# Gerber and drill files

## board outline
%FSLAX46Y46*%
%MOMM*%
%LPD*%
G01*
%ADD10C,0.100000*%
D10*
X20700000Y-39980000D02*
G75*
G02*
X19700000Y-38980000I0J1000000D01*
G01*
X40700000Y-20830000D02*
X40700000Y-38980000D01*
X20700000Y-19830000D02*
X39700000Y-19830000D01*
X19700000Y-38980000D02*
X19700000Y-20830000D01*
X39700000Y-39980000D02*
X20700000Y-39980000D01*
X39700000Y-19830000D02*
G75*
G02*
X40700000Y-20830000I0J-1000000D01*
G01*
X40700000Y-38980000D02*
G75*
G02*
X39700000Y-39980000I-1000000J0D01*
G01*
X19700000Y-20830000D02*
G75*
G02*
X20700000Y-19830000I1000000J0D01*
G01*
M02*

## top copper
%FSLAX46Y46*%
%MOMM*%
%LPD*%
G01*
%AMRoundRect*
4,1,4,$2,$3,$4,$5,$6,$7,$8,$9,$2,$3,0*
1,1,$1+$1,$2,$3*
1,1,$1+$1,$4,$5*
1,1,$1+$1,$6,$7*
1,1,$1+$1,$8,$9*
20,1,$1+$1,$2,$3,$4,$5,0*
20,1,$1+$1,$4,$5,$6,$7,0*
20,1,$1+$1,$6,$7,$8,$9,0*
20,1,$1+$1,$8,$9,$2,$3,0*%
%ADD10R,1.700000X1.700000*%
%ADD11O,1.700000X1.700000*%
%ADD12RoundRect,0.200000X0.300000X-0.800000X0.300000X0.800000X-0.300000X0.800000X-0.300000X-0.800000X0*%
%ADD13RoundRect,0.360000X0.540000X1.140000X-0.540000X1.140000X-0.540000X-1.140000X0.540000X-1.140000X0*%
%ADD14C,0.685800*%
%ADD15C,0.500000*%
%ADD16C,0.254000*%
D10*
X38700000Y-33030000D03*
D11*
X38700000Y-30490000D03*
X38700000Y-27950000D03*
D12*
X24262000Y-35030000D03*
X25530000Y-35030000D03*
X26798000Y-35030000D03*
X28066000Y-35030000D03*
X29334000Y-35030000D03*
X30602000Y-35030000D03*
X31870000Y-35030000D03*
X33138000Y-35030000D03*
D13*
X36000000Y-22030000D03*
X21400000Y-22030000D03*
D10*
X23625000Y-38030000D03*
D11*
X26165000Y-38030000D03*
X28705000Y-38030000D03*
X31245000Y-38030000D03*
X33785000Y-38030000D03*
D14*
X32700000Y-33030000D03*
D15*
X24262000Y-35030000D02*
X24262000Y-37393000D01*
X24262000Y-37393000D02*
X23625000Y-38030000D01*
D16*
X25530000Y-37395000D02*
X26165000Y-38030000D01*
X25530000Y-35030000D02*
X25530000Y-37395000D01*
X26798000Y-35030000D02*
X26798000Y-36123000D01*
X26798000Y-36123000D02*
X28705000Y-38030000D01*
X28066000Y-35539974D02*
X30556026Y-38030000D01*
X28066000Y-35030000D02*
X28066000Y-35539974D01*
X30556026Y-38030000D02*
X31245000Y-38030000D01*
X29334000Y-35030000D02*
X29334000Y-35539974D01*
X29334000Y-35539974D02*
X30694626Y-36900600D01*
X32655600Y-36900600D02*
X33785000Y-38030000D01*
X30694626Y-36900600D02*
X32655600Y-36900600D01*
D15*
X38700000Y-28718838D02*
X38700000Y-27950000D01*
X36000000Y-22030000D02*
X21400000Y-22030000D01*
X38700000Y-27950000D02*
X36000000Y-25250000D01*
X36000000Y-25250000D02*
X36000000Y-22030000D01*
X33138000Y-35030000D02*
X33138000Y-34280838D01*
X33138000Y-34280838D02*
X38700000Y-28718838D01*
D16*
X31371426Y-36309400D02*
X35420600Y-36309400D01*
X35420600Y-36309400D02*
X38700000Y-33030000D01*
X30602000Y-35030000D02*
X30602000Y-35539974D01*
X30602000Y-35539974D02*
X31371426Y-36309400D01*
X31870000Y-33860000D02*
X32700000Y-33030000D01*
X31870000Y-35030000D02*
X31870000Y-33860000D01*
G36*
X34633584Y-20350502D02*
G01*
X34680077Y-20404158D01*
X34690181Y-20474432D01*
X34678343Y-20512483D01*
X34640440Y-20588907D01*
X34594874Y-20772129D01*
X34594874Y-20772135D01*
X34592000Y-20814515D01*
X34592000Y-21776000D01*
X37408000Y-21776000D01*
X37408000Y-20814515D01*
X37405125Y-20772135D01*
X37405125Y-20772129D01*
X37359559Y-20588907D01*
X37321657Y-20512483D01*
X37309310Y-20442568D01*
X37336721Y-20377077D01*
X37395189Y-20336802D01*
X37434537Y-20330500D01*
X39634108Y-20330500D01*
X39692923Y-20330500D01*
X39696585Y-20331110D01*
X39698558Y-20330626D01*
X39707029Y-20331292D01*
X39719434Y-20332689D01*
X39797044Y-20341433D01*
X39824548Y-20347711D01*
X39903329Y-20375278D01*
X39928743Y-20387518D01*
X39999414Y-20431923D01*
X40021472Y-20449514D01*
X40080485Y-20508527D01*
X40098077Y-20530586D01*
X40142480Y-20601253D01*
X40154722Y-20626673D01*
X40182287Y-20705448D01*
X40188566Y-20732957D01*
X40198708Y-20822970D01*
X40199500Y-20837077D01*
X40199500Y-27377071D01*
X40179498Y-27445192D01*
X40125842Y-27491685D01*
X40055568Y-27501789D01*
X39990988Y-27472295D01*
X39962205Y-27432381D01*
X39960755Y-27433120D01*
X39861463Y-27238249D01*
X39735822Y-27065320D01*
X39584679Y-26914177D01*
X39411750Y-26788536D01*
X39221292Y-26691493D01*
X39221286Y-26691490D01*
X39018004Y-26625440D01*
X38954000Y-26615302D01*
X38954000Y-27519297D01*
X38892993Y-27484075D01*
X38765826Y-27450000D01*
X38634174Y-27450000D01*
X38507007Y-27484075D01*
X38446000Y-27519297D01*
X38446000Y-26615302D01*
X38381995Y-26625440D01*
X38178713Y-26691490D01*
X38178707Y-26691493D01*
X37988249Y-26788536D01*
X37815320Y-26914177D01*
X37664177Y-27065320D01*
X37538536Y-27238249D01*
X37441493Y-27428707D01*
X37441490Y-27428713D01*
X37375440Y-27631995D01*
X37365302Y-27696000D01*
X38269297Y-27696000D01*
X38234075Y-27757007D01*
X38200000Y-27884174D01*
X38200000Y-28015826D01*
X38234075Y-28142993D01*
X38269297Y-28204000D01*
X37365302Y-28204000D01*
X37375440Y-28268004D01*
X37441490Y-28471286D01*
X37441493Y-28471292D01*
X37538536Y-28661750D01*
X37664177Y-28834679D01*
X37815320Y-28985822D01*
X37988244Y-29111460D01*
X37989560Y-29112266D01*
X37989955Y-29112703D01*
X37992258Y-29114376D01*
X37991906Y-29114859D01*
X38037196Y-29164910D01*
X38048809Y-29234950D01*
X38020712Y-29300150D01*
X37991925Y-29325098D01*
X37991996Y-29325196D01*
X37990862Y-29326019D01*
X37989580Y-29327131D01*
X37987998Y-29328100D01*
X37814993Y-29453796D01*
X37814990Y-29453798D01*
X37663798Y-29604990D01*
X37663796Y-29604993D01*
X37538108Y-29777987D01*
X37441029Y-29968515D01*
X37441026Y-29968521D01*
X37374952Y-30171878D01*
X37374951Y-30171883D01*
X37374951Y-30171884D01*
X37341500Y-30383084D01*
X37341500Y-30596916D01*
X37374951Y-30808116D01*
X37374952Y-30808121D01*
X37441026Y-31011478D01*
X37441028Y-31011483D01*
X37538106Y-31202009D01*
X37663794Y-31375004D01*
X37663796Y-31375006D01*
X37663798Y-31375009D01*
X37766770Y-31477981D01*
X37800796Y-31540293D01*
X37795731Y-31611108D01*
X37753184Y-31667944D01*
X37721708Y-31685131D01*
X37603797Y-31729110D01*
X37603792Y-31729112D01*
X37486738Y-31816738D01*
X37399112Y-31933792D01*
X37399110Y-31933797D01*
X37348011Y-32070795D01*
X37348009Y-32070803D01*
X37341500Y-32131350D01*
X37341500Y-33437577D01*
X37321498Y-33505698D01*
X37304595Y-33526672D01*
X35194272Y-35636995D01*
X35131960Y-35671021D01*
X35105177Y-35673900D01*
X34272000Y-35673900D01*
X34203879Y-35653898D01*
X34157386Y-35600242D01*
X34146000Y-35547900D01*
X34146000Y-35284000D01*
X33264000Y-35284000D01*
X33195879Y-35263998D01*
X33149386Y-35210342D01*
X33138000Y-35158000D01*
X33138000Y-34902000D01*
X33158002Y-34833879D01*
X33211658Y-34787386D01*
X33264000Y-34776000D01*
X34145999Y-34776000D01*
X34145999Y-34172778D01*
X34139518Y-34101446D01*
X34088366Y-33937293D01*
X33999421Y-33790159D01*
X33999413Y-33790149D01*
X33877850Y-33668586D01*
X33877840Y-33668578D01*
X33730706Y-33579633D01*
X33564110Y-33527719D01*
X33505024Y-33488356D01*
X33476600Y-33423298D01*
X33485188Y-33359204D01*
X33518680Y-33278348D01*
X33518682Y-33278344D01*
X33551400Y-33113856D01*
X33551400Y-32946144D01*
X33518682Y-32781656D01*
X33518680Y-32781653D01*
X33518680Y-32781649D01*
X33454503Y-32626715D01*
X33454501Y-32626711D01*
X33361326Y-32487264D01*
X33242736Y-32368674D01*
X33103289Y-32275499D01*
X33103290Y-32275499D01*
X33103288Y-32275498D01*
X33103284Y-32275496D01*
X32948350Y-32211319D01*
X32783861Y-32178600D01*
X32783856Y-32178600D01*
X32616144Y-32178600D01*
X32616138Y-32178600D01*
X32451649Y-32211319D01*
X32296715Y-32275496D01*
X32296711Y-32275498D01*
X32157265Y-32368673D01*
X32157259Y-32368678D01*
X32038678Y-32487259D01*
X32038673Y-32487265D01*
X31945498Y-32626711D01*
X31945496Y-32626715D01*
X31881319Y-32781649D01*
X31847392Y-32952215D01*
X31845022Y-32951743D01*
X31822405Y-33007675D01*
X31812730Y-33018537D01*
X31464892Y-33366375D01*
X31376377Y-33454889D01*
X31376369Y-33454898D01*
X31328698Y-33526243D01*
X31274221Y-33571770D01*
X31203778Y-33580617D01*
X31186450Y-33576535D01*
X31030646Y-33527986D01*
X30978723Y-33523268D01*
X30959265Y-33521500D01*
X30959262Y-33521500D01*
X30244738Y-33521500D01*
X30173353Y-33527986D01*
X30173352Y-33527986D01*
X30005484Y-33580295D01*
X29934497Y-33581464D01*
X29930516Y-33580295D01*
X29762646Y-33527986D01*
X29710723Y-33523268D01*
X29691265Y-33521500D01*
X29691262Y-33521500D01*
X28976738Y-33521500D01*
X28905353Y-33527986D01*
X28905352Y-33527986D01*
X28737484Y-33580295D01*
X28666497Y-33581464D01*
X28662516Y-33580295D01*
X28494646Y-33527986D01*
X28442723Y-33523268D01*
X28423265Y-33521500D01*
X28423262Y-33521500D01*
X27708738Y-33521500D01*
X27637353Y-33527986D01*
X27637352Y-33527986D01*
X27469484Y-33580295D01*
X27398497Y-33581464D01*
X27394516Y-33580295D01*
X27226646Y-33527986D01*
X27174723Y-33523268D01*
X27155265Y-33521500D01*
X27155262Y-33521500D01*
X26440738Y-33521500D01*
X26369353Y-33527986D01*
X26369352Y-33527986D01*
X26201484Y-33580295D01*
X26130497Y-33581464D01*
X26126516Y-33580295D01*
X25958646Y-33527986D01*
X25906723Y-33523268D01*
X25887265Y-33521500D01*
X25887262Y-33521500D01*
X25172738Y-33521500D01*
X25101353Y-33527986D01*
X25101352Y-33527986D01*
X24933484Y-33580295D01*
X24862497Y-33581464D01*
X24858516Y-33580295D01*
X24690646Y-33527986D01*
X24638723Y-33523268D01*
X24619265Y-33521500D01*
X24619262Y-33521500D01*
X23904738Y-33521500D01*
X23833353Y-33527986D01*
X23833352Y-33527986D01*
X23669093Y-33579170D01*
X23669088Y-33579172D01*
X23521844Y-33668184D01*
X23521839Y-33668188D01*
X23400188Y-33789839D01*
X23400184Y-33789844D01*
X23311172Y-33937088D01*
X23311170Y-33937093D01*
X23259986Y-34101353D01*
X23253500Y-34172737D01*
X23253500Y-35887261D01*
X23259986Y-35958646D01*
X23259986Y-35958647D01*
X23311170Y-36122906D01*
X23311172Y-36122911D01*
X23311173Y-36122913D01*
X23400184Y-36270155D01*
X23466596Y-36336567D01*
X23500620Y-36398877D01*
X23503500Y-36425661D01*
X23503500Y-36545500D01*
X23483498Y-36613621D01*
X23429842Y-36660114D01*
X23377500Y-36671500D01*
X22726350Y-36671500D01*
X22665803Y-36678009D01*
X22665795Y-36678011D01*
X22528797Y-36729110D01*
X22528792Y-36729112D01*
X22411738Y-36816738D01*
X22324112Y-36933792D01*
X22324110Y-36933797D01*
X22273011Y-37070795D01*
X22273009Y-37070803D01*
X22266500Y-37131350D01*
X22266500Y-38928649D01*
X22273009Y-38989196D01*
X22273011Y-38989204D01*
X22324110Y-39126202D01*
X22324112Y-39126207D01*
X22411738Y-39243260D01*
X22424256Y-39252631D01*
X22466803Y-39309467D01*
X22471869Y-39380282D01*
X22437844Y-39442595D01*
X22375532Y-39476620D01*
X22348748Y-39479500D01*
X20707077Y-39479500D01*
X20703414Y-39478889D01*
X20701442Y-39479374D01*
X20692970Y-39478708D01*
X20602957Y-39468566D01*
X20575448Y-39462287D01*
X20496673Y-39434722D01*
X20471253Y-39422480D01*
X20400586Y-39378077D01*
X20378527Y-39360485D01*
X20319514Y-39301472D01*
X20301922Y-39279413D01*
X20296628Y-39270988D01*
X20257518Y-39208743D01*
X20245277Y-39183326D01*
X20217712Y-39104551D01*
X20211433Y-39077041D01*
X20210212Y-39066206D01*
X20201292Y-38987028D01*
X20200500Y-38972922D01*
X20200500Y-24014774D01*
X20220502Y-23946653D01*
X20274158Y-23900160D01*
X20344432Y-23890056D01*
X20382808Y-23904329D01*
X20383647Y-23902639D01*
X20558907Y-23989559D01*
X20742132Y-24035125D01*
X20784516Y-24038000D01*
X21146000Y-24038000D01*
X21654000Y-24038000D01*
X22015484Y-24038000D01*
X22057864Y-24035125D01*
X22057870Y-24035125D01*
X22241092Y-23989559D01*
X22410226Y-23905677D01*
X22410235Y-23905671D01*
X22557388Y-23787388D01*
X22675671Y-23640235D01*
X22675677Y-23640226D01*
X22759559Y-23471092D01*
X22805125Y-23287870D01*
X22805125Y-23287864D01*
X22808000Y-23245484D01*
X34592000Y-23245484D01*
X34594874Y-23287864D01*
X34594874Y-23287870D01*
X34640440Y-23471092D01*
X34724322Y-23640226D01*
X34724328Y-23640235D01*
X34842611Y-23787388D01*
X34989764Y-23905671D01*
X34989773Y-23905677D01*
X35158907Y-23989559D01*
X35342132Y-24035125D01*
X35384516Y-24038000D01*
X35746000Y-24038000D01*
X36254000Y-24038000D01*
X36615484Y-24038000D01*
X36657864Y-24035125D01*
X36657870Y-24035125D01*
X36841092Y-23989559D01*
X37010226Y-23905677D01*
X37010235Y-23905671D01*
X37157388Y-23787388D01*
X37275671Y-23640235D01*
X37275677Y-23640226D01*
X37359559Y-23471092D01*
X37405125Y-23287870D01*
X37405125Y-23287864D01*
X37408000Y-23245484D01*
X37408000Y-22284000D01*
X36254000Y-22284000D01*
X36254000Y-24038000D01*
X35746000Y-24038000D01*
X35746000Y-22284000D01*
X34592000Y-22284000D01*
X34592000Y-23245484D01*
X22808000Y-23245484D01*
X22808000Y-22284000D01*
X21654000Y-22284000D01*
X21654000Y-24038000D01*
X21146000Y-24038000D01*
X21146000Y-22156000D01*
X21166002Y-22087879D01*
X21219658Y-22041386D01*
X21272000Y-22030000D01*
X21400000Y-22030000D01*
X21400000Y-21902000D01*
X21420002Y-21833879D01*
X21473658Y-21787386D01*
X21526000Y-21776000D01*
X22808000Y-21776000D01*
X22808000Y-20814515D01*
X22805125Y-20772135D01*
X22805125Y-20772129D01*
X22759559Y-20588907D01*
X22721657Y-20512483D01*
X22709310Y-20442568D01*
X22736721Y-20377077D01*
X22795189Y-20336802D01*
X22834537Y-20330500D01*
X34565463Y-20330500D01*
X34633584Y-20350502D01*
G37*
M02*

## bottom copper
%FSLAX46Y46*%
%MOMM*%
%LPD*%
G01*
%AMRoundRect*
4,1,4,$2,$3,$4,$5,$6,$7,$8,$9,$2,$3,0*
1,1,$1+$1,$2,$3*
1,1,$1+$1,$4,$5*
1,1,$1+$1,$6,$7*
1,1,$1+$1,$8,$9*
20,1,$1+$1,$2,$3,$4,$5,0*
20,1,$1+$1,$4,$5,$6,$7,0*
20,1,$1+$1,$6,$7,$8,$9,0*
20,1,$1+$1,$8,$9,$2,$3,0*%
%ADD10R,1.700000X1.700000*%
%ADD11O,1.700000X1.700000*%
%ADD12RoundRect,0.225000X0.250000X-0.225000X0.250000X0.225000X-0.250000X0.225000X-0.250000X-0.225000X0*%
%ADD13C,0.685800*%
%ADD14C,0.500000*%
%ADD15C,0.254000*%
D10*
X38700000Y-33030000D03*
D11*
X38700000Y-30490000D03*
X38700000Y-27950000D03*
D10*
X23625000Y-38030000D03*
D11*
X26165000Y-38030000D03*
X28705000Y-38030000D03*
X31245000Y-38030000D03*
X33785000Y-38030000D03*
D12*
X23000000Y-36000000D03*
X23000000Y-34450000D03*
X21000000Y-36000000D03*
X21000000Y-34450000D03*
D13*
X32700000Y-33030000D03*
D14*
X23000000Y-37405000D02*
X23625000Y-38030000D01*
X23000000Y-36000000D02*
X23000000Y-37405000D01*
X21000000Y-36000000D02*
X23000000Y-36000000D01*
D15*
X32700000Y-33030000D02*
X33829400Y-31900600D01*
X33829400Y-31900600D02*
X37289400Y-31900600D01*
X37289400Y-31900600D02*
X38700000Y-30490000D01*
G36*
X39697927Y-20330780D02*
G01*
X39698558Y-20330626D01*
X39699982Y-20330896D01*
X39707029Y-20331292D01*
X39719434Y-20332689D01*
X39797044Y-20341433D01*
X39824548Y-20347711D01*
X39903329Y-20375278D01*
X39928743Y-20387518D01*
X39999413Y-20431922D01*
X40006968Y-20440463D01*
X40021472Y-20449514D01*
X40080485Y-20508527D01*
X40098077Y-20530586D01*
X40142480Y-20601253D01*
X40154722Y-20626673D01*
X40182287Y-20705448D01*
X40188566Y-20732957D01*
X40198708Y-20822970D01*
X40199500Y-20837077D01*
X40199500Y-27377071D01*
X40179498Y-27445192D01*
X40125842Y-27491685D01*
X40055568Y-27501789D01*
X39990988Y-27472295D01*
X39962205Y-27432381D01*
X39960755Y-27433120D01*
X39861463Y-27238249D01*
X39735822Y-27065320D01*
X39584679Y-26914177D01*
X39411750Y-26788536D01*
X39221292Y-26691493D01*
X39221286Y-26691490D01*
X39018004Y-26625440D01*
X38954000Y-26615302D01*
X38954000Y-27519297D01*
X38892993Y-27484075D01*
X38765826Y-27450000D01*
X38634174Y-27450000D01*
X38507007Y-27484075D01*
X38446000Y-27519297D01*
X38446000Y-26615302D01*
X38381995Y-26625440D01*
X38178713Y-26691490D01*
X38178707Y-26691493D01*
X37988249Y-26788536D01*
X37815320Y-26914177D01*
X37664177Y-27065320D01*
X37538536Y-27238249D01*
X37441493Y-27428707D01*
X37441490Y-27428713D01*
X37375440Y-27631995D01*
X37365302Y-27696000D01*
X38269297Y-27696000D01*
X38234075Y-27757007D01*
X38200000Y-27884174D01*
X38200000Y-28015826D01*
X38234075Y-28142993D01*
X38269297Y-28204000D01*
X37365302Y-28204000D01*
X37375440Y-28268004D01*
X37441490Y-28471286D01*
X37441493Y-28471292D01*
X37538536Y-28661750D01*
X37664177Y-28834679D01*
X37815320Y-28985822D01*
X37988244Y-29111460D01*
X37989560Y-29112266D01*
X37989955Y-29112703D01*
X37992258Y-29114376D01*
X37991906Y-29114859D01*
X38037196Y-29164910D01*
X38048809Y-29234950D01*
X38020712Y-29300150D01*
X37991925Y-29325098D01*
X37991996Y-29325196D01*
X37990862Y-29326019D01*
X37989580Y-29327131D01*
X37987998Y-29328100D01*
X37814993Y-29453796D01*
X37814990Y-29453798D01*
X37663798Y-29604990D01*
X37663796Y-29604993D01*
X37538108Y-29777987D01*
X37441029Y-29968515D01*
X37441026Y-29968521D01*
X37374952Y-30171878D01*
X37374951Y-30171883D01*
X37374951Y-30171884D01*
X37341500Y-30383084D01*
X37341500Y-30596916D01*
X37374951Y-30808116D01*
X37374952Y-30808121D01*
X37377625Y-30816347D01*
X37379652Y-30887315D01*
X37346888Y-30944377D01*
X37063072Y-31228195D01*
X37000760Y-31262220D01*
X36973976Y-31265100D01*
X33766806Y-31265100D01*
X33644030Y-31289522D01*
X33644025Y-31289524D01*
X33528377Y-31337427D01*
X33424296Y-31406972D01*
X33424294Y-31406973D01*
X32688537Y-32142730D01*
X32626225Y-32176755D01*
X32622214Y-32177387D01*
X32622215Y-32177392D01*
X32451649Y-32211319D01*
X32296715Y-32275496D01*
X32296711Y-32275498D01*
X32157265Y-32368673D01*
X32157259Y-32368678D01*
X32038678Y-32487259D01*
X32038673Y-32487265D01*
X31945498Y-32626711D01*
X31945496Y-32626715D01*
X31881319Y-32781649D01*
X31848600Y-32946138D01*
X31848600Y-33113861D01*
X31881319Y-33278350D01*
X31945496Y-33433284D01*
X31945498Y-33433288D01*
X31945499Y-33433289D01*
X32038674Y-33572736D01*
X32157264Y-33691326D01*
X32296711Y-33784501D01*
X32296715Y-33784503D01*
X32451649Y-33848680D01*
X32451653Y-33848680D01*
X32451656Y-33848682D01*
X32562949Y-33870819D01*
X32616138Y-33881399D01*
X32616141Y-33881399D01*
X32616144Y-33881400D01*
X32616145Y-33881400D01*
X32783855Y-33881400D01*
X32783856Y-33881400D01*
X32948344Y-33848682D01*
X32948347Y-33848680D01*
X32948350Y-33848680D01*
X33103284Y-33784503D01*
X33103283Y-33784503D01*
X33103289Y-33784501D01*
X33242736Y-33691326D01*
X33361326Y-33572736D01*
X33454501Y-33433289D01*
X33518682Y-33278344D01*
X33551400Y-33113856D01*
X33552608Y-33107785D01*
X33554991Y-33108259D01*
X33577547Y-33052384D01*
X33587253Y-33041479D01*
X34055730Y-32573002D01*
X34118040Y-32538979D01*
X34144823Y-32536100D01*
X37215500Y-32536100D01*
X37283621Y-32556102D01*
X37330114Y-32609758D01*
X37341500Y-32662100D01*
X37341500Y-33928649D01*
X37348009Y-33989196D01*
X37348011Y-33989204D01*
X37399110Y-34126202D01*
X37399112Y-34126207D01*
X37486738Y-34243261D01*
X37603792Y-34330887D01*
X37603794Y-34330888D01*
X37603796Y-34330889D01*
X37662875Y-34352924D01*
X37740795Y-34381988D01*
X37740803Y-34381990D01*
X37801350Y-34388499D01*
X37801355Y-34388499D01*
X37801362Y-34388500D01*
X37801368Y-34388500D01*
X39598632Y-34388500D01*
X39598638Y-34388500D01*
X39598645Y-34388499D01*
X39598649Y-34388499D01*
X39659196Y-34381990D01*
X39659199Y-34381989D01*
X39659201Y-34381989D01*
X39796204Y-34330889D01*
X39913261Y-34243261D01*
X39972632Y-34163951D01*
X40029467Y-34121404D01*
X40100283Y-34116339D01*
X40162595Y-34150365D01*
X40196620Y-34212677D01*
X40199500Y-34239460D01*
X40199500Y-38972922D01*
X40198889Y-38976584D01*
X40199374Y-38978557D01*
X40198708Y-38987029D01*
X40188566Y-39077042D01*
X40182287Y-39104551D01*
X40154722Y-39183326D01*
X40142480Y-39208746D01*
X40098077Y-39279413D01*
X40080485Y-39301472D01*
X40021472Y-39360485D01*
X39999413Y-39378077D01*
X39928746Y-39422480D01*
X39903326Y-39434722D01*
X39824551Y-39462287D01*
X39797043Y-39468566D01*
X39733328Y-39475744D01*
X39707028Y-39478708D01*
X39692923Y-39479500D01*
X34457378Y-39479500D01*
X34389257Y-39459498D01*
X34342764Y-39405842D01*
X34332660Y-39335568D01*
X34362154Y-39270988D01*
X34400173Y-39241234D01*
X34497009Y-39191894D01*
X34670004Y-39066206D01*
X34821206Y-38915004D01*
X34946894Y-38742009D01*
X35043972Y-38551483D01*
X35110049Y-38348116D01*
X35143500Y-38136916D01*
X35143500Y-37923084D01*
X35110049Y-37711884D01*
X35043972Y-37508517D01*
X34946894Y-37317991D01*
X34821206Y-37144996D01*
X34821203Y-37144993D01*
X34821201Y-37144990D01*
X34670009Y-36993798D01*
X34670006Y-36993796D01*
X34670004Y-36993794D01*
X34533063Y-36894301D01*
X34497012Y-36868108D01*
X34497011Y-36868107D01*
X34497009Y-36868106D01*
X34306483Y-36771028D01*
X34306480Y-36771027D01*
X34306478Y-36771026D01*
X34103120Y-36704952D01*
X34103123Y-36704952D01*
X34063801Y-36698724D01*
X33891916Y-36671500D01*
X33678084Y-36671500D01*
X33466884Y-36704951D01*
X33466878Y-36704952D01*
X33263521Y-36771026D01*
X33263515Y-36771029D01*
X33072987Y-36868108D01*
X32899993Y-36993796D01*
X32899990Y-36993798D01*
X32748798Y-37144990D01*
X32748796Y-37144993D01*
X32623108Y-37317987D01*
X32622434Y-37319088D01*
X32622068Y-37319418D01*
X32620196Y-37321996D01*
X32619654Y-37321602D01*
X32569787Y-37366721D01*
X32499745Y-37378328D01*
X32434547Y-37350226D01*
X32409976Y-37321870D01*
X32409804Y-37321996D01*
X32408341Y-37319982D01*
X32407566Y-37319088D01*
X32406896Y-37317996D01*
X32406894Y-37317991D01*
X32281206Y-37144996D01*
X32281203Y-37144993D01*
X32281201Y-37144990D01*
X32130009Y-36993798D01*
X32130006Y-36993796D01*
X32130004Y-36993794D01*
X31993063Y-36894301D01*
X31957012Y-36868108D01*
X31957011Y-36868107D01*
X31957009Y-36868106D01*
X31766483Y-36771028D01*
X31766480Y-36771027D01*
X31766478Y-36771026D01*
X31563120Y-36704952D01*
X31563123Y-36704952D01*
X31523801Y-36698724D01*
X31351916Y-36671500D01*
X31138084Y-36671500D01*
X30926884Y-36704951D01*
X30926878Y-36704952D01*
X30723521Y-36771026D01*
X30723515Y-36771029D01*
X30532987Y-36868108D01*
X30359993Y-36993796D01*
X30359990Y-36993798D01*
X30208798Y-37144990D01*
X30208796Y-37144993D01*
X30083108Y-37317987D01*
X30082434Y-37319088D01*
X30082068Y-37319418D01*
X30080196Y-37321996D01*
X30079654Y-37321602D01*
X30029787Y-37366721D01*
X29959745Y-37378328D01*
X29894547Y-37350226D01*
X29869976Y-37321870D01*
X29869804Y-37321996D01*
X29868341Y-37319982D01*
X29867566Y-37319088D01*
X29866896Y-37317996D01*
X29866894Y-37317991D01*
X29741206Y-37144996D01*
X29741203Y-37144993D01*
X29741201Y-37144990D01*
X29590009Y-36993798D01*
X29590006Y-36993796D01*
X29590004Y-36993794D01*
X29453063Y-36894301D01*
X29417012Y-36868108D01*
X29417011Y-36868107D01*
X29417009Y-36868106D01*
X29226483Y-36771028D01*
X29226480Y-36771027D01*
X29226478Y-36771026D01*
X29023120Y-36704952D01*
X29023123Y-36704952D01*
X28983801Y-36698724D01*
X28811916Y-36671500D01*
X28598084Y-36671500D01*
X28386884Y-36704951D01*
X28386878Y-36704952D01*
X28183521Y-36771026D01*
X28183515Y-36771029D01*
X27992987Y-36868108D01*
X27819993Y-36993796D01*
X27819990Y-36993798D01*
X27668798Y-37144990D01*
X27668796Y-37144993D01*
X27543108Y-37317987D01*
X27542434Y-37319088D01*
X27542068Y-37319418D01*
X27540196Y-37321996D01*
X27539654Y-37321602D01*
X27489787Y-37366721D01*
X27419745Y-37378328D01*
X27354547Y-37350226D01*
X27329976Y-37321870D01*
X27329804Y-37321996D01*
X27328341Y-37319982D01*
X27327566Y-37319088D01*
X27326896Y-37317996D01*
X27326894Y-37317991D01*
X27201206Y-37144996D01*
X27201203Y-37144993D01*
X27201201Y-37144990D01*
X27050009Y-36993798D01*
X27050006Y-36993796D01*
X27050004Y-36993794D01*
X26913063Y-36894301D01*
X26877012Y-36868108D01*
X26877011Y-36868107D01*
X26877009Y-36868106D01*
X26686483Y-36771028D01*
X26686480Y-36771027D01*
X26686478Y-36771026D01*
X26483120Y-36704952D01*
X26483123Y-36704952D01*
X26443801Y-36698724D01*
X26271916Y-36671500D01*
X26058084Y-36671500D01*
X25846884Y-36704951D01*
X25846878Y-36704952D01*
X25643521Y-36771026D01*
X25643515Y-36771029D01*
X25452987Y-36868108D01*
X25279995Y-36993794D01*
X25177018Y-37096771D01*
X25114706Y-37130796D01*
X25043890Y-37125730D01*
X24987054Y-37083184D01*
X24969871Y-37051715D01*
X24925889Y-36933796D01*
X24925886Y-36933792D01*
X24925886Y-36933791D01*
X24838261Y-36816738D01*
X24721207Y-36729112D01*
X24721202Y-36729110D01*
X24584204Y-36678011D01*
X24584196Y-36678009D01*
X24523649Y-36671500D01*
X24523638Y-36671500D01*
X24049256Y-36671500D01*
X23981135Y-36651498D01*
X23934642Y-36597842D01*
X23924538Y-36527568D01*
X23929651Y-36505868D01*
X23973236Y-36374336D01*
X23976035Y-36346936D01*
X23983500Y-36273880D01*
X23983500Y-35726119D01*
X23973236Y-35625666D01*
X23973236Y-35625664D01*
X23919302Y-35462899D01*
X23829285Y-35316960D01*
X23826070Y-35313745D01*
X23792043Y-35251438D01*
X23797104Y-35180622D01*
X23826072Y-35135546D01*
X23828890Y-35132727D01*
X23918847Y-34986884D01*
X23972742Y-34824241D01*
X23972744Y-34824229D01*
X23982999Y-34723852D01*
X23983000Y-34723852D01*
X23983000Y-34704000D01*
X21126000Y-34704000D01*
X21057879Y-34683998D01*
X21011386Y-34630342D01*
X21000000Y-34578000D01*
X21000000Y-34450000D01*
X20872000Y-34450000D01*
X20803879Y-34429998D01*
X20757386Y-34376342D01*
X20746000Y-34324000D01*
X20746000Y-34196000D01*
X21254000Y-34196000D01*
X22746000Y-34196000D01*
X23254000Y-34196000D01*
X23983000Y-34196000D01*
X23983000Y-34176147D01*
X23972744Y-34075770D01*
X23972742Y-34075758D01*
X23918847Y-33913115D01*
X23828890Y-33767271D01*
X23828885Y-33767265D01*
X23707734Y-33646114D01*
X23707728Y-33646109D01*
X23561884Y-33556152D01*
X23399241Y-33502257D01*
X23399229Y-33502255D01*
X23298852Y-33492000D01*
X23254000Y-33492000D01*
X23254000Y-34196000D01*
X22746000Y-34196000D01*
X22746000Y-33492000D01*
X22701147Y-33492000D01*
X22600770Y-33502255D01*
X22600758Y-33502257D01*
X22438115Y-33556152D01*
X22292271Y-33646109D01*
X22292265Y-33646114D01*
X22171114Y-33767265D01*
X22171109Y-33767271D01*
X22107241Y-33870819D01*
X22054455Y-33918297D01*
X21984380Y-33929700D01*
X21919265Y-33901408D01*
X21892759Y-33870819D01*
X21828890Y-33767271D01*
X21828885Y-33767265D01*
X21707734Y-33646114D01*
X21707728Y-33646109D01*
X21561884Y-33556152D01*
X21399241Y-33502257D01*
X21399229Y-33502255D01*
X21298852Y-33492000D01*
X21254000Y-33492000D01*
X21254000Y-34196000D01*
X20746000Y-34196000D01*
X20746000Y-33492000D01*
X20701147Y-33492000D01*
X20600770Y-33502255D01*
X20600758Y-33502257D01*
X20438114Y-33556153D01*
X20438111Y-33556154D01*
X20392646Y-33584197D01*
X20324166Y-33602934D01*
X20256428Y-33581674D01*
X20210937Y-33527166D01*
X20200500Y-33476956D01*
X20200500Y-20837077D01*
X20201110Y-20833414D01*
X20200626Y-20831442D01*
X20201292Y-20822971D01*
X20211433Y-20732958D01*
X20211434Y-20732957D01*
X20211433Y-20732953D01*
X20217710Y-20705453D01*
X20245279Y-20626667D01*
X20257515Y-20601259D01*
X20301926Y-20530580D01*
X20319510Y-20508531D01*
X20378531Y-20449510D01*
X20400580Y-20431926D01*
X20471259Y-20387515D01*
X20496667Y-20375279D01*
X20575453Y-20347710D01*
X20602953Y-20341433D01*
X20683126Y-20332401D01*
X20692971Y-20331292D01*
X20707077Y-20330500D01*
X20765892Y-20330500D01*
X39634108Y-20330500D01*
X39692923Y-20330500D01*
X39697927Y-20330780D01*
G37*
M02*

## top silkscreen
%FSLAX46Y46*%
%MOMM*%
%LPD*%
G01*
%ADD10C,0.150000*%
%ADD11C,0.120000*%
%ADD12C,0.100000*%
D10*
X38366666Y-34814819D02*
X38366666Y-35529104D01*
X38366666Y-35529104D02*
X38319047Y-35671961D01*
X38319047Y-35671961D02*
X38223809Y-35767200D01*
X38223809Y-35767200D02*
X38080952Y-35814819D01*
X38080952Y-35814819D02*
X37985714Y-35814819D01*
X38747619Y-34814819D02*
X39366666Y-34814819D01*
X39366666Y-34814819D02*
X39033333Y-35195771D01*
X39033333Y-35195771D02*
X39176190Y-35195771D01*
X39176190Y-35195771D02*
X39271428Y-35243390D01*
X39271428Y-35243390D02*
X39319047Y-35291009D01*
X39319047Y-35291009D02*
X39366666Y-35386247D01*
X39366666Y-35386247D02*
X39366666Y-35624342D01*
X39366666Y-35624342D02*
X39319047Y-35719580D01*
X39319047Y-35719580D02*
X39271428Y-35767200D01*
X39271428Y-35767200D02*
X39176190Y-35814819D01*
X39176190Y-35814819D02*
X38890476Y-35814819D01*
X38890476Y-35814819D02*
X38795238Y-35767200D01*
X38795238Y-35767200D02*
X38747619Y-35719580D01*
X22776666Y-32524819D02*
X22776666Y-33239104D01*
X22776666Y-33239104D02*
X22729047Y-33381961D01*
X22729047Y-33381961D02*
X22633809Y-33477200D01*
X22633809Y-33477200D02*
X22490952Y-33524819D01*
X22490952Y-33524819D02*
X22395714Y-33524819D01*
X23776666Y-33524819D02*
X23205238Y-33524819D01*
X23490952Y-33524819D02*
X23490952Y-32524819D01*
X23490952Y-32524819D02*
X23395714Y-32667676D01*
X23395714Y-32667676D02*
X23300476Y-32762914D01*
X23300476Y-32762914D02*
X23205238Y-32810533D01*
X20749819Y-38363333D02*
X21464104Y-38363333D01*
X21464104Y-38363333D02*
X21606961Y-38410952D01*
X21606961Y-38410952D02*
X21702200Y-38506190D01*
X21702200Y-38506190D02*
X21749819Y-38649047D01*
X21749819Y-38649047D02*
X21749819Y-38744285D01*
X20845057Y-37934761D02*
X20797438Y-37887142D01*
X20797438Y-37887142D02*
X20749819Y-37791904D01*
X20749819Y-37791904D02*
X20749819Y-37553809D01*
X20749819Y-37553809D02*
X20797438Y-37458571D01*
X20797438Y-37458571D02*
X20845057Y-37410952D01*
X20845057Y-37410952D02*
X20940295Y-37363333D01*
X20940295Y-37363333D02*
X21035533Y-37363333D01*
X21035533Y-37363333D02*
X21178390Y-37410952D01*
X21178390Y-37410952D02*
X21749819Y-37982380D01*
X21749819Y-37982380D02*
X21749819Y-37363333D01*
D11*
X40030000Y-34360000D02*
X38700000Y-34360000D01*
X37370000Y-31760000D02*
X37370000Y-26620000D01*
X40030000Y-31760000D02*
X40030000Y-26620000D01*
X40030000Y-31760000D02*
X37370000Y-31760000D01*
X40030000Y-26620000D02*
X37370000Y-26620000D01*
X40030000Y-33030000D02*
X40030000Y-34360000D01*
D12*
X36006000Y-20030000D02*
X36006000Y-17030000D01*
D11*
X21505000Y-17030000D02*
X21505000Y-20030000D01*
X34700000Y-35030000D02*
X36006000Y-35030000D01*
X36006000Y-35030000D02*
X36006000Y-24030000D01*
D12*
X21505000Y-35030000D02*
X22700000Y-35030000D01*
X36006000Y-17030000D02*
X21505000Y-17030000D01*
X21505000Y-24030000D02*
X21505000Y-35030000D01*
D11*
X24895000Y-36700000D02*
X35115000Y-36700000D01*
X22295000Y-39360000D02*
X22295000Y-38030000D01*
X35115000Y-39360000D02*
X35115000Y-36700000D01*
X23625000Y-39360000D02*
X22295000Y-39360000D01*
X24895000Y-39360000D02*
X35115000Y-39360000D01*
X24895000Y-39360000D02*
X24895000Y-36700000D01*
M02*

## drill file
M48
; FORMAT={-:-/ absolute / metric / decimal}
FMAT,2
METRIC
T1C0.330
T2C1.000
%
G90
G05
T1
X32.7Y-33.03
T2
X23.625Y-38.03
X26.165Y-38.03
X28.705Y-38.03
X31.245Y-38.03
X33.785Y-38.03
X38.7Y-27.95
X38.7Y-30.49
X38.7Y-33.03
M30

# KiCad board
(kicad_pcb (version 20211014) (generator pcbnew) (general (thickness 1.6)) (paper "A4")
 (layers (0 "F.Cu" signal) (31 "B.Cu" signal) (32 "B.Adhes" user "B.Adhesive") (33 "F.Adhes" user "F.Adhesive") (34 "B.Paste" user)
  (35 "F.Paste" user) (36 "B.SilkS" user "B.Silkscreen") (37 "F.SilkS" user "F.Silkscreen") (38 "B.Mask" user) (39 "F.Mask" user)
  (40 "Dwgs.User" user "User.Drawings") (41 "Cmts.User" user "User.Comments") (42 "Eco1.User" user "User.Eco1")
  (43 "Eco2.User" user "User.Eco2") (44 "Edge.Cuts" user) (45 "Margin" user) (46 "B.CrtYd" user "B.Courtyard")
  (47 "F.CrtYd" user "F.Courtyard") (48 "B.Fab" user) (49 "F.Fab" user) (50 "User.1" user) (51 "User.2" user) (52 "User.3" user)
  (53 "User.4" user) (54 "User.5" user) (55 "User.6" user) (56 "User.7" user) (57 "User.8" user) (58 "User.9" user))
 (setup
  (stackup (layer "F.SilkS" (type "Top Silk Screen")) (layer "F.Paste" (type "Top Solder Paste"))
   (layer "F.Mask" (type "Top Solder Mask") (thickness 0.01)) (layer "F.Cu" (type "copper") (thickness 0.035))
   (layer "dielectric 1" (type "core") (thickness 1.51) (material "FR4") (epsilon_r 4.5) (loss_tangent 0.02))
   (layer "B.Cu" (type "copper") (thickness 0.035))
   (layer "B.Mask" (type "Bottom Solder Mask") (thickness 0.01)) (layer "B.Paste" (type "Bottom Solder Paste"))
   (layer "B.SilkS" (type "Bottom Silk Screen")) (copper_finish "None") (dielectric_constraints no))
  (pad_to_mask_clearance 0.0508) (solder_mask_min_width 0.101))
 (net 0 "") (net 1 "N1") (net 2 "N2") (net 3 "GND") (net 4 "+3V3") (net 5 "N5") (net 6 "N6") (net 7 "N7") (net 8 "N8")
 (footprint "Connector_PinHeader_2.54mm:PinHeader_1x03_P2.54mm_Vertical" (layer "F.Cu") (at 38.7 33.03 180)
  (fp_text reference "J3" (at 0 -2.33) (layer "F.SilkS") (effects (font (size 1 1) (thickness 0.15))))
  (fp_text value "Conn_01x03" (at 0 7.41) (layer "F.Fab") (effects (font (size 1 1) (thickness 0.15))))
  (fp_line (start -1.33 -1.33) (end 0 -1.33) (layer "F.SilkS") (width 0.12))
  (fp_line (start 1.33 1.27) (end 1.33 6.41) (layer "F.SilkS") (width 0.12))
  (fp_line (start -1.33 1.27) (end -1.33 6.41) (layer "F.SilkS") (width 0.12))
  (fp_line (start -1.33 1.27) (end 1.33 1.27) (layer "F.SilkS") (width 0.12))
  (fp_line (start -1.33 6.41) (end 1.33 6.41) (layer "F.SilkS") (width 0.12))
  (fp_line (start -1.33 0) (end -1.33 -1.33) (layer "F.SilkS") (width 0.12))
  (pad "1" thru_hole rect (at 0 0 180) (size 1.7 1.7) (drill 1) (layers *.Cu *.Mask) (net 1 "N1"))
  (pad "2" thru_hole oval (at 0 2.54 180) (size 1.7 1.7) (drill 1) (layers *.Cu *.Mask) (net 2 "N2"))
  (pad "3" thru_hole oval (at 0 5.08 180) (size 1.7 1.7) (drill 1) (layers *.Cu *.Mask) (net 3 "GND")))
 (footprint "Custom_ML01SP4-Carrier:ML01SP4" (layer "F.Cu") (at 28.7 35.03)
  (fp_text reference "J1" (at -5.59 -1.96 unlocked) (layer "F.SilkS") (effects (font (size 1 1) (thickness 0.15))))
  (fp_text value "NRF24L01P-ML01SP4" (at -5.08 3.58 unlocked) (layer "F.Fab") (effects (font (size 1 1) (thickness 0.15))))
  (fp_line (start 7.306 -15) (end 7.306 -18) (layer "F.SilkS") (width 0.1))
  (fp_line (start -7.195 -18) (end -7.195 -15) (layer "F.SilkS") (width 0.12))
  (fp_line (start 6 0) (end 7.306 0) (layer "F.SilkS") (width 0.12))
  (fp_line (start 7.306 0) (end 7.306 -11) (layer "F.SilkS") (width 0.12))
  (fp_line (start -7.195 0) (end -6 0) (layer "F.SilkS") (width 0.1))
  (fp_line (start 7.306 -18) (end -7.195 -18) (layer "F.SilkS") (width 0.1))
  (fp_line (start -7.195 -11) (end -7.195 0) (layer "F.SilkS") (width 0.1))
  (pad "1" smd roundrect (at -4.438 0 90) (size 2 1) (layers "F.Cu" "F.Paste" "F.Mask") (roundrect_rratio 0.2) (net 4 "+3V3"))
  (pad "2" smd roundrect (at -3.17 0 90) (size 2 1) (layers "F.Cu" "F.Paste" "F.Mask") (roundrect_rratio 0.2) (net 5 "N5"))
  (pad "3" smd roundrect (at -1.902 0 90) (size 2 1) (layers "F.Cu" "F.Paste" "F.Mask") (roundrect_rratio 0.2) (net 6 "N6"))
  (pad "4" smd roundrect (at -0.634 0 90) (size 2 1) (layers "F.Cu" "F.Paste" "F.Mask") (roundrect_rratio 0.2) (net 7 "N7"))
  (pad "5" smd roundrect (at 0.634 0 90) (size 2 1) (layers "F.Cu" "F.Paste" "F.Mask") (roundrect_rratio 0.2) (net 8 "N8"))
  (pad "6" smd roundrect (at 1.902 0 90) (size 2 1) (layers "F.Cu" "F.Paste" "F.Mask") (roundrect_rratio 0.2) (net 1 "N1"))
  (pad "7" smd roundrect (at 3.17 0 90) (size 2 1) (layers "F.Cu" "F.Paste" "F.Mask") (roundrect_rratio 0.2) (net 2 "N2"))
  (pad "8" smd roundrect (at 4.438 0 90) (size 2 1) (layers "F.Cu" "F.Paste" "F.Mask") (roundrect_rratio 0.2) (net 3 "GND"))
  (pad "9" smd roundrect (at 7.3 -13 180) (size 1.8 3) (layers "F.Cu" "F.Paste" "F.Mask") (roundrect_rratio 0.2) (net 3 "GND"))
  (pad "10" smd roundrect (at -7.3 -13 180) (size 1.8 3) (layers "F.Cu" "F.Paste" "F.Mask") (roundrect_rratio 0.2) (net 3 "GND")))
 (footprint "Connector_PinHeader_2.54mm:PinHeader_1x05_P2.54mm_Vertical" (layer "F.Cu") (at 23.625 38.03 90)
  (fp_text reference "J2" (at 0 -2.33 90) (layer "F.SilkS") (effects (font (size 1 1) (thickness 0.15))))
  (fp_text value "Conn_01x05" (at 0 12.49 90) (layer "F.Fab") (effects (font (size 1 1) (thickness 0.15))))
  (fp_line (start 1.33 1.27) (end 1.33 11.49) (layer "F.SilkS") (width 0.12))
  (fp_line (start -1.33 -1.33) (end 0 -1.33) (layer "F.SilkS") (width 0.12))
  (fp_line (start -1.33 11.49) (end 1.33 11.49) (layer "F.SilkS") (width 0.12))
  (fp_line (start -1.33 0) (end -1.33 -1.33) (layer "F.SilkS") (width 0.12))
  (fp_line (start -1.33 1.27) (end -1.33 11.49) (layer "F.SilkS") (width 0.12))
  (fp_line (start -1.33 1.27) (end 1.33 1.27) (layer "F.SilkS") (width 0.12))
  (pad "1" thru_hole rect (at 0 0 90) (size 1.7 1.7) (drill 1) (layers *.Cu *.Mask) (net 4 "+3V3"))
  (pad "2" thru_hole oval (at 0 2.54 90) (size 1.7 1.7) (drill 1) (layers *.Cu *.Mask) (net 5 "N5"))
  (pad "3" thru_hole oval (at 0 5.08 90) (size 1.7 1.7) (drill 1) (layers *.Cu *.Mask) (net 6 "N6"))
  (pad "4" thru_hole oval (at 0 7.62 90) (size 1.7 1.7) (drill 1) (layers *.Cu *.Mask) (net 7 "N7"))
  (pad "5" thru_hole oval (at 0 10.16 90) (size 1.7 1.7) (drill 1) (layers *.Cu *.Mask) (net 8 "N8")))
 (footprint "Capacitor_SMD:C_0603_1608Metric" (layer "B.Cu") (at 23 35.225 90)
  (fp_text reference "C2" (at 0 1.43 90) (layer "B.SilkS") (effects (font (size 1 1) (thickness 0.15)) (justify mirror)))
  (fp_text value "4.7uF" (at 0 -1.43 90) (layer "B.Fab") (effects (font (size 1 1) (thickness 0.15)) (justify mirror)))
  (pad "1" smd roundrect (at -0.775 0 90) (size 0.9 0.95) (layers "B.Cu" "B.Paste" "B.Mask") (roundrect_rratio 0.25) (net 4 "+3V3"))
  (pad "2" smd roundrect (at 0.775 0 90) (size 0.9 0.95) (layers "B.Cu" "B.Paste" "B.Mask") (roundrect_rratio 0.25) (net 3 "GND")))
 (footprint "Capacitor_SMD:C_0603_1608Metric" (layer "B.Cu") (at 21 35.225 90)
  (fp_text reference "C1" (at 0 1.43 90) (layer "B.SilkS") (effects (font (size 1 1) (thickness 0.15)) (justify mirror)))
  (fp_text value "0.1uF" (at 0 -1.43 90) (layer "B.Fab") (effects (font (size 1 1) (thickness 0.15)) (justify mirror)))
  (pad "1" smd roundrect (at -0.775 0 90) (size 0.9 0.95) (layers "B.Cu" "B.Paste" "B.Mask") (roundrect_rratio 0.25) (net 4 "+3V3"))
  (pad "2" smd roundrect (at 0.775 0 90) (size 0.9 0.95) (layers "B.Cu" "B.Paste" "B.Mask") (roundrect_rratio 0.25) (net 3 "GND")))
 (gr_arc (start 20.7 39.98) (mid 19.992893 39.687107) (end 19.7 38.98) (layer "Edge.Cuts") (width 0.1))
 (gr_line (start 40.7 20.83) (end 40.7 38.98) (layer "Edge.Cuts") (width 0.1))
 (gr_line (start 20.7 19.83) (end 39.7 19.83) (layer "Edge.Cuts") (width 0.1))
 (gr_line (start 19.7 38.98) (end 19.7 20.83) (layer "Edge.Cuts") (width 0.1))
 (gr_line (start 39.7 39.98) (end 20.7 39.98) (layer "Edge.Cuts") (width 0.1))
 (gr_arc (start 39.7 19.83) (mid 40.407107 20.122893) (end 40.7 20.83) (layer "Edge.Cuts") (width 0.1))
 (gr_arc (start 40.7 38.98) (mid 40.407107 39.687107) (end 39.7 39.98) (layer "Edge.Cuts") (width 0.1))
 (gr_arc (start 19.7 20.83) (mid 19.992893 20.122893) (end 20.7 19.83) (layer "Edge.Cuts") (width 0.1))
 (segment (start 24.262 35.03) (end 24.262 37.393) (width 0.5) (layer "F.Cu") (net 4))
 (segment (start 24.262 37.393) (end 23.625 38.03) (width 0.5) (layer "F.Cu") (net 4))
 (segment (start 23 37.405) (end 23.625 38.03) (width 0.5) (layer "B.Cu") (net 4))
 (segment (start 23 36) (end 23 37.405) (width 0.5) (layer "B.Cu") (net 4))
 (segment (start 21 36) (end 23 36) (width 0.5) (layer "B.Cu") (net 4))
 (segment (start 25.53 37.395) (end 26.165 38.03) (width 0.254) (layer "F.Cu") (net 5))
 (segment (start 25.53 35.03) (end 25.53 37.395) (width 0.254) (layer "F.Cu") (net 5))
 (segment (start 26.798 35.03) (end 26.798 36.123) (width 0.254) (layer "F.Cu") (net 6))
 (segment (start 26.798 36.123) (end 28.705 38.03) (width 0.254) (layer "F.Cu") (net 6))
 (segment (start 28.066 35.539974) (end 30.556026 38.03) (width 0.254) (layer "F.Cu") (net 7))
 (segment (start 28.066 35.03) (end 28.066 35.539974) (width 0.254) (layer "F.Cu") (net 7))
 (segment (start 30.556026 38.03) (end 31.245 38.03) (width 0.254) (layer "F.Cu") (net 7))
 (segment (start 29.334 35.03) (end 29.334 35.539974) (width 0.254) (layer "F.Cu") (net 8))
 (segment (start 29.334 35.539974) (end 30.694626 36.9006) (width 0.254) (layer "F.Cu") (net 8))
 (segment (start 32.6556 36.9006) (end 33.785 38.03) (width 0.254) (layer "F.Cu") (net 8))
 (segment (start 30.694626 36.9006) (end 32.6556 36.9006) (width 0.254) (layer "F.Cu") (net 8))
 (segment (start 38.7 28.718838) (end 38.7 27.95) (width 0.5) (layer "F.Cu") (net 3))
 (segment (start 36 22.03) (end 21.4 22.03) (width 0.5) (layer "F.Cu") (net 3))
 (segment (start 38.7 27.95) (end 36 25.25) (width 0.5) (layer "F.Cu") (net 3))
 (segment (start 36 25.25) (end 36 22.03) (width 0.5) (layer "F.Cu") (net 3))
 (segment (start 33.138 35.03) (end 33.138 34.280838) (width 0.5) (layer "F.Cu") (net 3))
 (segment (start 33.138 34.280838) (end 38.7 28.718838) (width 0.5) (layer "F.Cu") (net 3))
 (segment (start 31.371426 36.3094) (end 35.4206 36.3094) (width 0.254) (layer "F.Cu") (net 1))
 (segment (start 35.4206 36.3094) (end 38.7 33.03) (width 0.254) (layer "F.Cu") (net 1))
 (segment (start 30.602 35.03) (end 30.602 35.539974) (width 0.254) (layer "F.Cu") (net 1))
 (segment (start 30.602 35.539974) (end 31.371426 36.3094) (width 0.254) (layer "F.Cu") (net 1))
 (segment (start 31.87 33.86) (end 32.7 33.03) (width 0.254) (layer "F.Cu") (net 2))
 (segment (start 31.87 35.03) (end 31.87 33.86) (width 0.254) (layer "F.Cu") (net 2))
 (via (at 32.7 33.03) (size 0.6858) (drill 0.3302) (layers "F.Cu" "B.Cu") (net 2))
 (segment (start 32.7 33.03) (end 33.8294 31.9006) (width 0.254) (layer "B.Cu") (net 2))
 (segment (start 33.8294 31.9006) (end 37.2894 31.9006) (width 0.254) (layer "B.Cu") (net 2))
 (segment (start 37.2894 31.9006) (end 38.7 30.49) (width 0.254) (layer "B.Cu") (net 2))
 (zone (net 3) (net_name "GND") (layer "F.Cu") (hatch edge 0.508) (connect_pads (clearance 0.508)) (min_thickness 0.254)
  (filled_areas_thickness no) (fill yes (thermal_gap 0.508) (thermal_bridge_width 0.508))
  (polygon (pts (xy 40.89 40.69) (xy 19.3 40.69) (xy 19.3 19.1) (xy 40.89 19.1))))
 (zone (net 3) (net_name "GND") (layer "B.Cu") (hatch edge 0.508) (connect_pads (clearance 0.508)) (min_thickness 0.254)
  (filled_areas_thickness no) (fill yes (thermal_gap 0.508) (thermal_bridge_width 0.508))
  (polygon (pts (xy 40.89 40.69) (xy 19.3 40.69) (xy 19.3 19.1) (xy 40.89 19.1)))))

